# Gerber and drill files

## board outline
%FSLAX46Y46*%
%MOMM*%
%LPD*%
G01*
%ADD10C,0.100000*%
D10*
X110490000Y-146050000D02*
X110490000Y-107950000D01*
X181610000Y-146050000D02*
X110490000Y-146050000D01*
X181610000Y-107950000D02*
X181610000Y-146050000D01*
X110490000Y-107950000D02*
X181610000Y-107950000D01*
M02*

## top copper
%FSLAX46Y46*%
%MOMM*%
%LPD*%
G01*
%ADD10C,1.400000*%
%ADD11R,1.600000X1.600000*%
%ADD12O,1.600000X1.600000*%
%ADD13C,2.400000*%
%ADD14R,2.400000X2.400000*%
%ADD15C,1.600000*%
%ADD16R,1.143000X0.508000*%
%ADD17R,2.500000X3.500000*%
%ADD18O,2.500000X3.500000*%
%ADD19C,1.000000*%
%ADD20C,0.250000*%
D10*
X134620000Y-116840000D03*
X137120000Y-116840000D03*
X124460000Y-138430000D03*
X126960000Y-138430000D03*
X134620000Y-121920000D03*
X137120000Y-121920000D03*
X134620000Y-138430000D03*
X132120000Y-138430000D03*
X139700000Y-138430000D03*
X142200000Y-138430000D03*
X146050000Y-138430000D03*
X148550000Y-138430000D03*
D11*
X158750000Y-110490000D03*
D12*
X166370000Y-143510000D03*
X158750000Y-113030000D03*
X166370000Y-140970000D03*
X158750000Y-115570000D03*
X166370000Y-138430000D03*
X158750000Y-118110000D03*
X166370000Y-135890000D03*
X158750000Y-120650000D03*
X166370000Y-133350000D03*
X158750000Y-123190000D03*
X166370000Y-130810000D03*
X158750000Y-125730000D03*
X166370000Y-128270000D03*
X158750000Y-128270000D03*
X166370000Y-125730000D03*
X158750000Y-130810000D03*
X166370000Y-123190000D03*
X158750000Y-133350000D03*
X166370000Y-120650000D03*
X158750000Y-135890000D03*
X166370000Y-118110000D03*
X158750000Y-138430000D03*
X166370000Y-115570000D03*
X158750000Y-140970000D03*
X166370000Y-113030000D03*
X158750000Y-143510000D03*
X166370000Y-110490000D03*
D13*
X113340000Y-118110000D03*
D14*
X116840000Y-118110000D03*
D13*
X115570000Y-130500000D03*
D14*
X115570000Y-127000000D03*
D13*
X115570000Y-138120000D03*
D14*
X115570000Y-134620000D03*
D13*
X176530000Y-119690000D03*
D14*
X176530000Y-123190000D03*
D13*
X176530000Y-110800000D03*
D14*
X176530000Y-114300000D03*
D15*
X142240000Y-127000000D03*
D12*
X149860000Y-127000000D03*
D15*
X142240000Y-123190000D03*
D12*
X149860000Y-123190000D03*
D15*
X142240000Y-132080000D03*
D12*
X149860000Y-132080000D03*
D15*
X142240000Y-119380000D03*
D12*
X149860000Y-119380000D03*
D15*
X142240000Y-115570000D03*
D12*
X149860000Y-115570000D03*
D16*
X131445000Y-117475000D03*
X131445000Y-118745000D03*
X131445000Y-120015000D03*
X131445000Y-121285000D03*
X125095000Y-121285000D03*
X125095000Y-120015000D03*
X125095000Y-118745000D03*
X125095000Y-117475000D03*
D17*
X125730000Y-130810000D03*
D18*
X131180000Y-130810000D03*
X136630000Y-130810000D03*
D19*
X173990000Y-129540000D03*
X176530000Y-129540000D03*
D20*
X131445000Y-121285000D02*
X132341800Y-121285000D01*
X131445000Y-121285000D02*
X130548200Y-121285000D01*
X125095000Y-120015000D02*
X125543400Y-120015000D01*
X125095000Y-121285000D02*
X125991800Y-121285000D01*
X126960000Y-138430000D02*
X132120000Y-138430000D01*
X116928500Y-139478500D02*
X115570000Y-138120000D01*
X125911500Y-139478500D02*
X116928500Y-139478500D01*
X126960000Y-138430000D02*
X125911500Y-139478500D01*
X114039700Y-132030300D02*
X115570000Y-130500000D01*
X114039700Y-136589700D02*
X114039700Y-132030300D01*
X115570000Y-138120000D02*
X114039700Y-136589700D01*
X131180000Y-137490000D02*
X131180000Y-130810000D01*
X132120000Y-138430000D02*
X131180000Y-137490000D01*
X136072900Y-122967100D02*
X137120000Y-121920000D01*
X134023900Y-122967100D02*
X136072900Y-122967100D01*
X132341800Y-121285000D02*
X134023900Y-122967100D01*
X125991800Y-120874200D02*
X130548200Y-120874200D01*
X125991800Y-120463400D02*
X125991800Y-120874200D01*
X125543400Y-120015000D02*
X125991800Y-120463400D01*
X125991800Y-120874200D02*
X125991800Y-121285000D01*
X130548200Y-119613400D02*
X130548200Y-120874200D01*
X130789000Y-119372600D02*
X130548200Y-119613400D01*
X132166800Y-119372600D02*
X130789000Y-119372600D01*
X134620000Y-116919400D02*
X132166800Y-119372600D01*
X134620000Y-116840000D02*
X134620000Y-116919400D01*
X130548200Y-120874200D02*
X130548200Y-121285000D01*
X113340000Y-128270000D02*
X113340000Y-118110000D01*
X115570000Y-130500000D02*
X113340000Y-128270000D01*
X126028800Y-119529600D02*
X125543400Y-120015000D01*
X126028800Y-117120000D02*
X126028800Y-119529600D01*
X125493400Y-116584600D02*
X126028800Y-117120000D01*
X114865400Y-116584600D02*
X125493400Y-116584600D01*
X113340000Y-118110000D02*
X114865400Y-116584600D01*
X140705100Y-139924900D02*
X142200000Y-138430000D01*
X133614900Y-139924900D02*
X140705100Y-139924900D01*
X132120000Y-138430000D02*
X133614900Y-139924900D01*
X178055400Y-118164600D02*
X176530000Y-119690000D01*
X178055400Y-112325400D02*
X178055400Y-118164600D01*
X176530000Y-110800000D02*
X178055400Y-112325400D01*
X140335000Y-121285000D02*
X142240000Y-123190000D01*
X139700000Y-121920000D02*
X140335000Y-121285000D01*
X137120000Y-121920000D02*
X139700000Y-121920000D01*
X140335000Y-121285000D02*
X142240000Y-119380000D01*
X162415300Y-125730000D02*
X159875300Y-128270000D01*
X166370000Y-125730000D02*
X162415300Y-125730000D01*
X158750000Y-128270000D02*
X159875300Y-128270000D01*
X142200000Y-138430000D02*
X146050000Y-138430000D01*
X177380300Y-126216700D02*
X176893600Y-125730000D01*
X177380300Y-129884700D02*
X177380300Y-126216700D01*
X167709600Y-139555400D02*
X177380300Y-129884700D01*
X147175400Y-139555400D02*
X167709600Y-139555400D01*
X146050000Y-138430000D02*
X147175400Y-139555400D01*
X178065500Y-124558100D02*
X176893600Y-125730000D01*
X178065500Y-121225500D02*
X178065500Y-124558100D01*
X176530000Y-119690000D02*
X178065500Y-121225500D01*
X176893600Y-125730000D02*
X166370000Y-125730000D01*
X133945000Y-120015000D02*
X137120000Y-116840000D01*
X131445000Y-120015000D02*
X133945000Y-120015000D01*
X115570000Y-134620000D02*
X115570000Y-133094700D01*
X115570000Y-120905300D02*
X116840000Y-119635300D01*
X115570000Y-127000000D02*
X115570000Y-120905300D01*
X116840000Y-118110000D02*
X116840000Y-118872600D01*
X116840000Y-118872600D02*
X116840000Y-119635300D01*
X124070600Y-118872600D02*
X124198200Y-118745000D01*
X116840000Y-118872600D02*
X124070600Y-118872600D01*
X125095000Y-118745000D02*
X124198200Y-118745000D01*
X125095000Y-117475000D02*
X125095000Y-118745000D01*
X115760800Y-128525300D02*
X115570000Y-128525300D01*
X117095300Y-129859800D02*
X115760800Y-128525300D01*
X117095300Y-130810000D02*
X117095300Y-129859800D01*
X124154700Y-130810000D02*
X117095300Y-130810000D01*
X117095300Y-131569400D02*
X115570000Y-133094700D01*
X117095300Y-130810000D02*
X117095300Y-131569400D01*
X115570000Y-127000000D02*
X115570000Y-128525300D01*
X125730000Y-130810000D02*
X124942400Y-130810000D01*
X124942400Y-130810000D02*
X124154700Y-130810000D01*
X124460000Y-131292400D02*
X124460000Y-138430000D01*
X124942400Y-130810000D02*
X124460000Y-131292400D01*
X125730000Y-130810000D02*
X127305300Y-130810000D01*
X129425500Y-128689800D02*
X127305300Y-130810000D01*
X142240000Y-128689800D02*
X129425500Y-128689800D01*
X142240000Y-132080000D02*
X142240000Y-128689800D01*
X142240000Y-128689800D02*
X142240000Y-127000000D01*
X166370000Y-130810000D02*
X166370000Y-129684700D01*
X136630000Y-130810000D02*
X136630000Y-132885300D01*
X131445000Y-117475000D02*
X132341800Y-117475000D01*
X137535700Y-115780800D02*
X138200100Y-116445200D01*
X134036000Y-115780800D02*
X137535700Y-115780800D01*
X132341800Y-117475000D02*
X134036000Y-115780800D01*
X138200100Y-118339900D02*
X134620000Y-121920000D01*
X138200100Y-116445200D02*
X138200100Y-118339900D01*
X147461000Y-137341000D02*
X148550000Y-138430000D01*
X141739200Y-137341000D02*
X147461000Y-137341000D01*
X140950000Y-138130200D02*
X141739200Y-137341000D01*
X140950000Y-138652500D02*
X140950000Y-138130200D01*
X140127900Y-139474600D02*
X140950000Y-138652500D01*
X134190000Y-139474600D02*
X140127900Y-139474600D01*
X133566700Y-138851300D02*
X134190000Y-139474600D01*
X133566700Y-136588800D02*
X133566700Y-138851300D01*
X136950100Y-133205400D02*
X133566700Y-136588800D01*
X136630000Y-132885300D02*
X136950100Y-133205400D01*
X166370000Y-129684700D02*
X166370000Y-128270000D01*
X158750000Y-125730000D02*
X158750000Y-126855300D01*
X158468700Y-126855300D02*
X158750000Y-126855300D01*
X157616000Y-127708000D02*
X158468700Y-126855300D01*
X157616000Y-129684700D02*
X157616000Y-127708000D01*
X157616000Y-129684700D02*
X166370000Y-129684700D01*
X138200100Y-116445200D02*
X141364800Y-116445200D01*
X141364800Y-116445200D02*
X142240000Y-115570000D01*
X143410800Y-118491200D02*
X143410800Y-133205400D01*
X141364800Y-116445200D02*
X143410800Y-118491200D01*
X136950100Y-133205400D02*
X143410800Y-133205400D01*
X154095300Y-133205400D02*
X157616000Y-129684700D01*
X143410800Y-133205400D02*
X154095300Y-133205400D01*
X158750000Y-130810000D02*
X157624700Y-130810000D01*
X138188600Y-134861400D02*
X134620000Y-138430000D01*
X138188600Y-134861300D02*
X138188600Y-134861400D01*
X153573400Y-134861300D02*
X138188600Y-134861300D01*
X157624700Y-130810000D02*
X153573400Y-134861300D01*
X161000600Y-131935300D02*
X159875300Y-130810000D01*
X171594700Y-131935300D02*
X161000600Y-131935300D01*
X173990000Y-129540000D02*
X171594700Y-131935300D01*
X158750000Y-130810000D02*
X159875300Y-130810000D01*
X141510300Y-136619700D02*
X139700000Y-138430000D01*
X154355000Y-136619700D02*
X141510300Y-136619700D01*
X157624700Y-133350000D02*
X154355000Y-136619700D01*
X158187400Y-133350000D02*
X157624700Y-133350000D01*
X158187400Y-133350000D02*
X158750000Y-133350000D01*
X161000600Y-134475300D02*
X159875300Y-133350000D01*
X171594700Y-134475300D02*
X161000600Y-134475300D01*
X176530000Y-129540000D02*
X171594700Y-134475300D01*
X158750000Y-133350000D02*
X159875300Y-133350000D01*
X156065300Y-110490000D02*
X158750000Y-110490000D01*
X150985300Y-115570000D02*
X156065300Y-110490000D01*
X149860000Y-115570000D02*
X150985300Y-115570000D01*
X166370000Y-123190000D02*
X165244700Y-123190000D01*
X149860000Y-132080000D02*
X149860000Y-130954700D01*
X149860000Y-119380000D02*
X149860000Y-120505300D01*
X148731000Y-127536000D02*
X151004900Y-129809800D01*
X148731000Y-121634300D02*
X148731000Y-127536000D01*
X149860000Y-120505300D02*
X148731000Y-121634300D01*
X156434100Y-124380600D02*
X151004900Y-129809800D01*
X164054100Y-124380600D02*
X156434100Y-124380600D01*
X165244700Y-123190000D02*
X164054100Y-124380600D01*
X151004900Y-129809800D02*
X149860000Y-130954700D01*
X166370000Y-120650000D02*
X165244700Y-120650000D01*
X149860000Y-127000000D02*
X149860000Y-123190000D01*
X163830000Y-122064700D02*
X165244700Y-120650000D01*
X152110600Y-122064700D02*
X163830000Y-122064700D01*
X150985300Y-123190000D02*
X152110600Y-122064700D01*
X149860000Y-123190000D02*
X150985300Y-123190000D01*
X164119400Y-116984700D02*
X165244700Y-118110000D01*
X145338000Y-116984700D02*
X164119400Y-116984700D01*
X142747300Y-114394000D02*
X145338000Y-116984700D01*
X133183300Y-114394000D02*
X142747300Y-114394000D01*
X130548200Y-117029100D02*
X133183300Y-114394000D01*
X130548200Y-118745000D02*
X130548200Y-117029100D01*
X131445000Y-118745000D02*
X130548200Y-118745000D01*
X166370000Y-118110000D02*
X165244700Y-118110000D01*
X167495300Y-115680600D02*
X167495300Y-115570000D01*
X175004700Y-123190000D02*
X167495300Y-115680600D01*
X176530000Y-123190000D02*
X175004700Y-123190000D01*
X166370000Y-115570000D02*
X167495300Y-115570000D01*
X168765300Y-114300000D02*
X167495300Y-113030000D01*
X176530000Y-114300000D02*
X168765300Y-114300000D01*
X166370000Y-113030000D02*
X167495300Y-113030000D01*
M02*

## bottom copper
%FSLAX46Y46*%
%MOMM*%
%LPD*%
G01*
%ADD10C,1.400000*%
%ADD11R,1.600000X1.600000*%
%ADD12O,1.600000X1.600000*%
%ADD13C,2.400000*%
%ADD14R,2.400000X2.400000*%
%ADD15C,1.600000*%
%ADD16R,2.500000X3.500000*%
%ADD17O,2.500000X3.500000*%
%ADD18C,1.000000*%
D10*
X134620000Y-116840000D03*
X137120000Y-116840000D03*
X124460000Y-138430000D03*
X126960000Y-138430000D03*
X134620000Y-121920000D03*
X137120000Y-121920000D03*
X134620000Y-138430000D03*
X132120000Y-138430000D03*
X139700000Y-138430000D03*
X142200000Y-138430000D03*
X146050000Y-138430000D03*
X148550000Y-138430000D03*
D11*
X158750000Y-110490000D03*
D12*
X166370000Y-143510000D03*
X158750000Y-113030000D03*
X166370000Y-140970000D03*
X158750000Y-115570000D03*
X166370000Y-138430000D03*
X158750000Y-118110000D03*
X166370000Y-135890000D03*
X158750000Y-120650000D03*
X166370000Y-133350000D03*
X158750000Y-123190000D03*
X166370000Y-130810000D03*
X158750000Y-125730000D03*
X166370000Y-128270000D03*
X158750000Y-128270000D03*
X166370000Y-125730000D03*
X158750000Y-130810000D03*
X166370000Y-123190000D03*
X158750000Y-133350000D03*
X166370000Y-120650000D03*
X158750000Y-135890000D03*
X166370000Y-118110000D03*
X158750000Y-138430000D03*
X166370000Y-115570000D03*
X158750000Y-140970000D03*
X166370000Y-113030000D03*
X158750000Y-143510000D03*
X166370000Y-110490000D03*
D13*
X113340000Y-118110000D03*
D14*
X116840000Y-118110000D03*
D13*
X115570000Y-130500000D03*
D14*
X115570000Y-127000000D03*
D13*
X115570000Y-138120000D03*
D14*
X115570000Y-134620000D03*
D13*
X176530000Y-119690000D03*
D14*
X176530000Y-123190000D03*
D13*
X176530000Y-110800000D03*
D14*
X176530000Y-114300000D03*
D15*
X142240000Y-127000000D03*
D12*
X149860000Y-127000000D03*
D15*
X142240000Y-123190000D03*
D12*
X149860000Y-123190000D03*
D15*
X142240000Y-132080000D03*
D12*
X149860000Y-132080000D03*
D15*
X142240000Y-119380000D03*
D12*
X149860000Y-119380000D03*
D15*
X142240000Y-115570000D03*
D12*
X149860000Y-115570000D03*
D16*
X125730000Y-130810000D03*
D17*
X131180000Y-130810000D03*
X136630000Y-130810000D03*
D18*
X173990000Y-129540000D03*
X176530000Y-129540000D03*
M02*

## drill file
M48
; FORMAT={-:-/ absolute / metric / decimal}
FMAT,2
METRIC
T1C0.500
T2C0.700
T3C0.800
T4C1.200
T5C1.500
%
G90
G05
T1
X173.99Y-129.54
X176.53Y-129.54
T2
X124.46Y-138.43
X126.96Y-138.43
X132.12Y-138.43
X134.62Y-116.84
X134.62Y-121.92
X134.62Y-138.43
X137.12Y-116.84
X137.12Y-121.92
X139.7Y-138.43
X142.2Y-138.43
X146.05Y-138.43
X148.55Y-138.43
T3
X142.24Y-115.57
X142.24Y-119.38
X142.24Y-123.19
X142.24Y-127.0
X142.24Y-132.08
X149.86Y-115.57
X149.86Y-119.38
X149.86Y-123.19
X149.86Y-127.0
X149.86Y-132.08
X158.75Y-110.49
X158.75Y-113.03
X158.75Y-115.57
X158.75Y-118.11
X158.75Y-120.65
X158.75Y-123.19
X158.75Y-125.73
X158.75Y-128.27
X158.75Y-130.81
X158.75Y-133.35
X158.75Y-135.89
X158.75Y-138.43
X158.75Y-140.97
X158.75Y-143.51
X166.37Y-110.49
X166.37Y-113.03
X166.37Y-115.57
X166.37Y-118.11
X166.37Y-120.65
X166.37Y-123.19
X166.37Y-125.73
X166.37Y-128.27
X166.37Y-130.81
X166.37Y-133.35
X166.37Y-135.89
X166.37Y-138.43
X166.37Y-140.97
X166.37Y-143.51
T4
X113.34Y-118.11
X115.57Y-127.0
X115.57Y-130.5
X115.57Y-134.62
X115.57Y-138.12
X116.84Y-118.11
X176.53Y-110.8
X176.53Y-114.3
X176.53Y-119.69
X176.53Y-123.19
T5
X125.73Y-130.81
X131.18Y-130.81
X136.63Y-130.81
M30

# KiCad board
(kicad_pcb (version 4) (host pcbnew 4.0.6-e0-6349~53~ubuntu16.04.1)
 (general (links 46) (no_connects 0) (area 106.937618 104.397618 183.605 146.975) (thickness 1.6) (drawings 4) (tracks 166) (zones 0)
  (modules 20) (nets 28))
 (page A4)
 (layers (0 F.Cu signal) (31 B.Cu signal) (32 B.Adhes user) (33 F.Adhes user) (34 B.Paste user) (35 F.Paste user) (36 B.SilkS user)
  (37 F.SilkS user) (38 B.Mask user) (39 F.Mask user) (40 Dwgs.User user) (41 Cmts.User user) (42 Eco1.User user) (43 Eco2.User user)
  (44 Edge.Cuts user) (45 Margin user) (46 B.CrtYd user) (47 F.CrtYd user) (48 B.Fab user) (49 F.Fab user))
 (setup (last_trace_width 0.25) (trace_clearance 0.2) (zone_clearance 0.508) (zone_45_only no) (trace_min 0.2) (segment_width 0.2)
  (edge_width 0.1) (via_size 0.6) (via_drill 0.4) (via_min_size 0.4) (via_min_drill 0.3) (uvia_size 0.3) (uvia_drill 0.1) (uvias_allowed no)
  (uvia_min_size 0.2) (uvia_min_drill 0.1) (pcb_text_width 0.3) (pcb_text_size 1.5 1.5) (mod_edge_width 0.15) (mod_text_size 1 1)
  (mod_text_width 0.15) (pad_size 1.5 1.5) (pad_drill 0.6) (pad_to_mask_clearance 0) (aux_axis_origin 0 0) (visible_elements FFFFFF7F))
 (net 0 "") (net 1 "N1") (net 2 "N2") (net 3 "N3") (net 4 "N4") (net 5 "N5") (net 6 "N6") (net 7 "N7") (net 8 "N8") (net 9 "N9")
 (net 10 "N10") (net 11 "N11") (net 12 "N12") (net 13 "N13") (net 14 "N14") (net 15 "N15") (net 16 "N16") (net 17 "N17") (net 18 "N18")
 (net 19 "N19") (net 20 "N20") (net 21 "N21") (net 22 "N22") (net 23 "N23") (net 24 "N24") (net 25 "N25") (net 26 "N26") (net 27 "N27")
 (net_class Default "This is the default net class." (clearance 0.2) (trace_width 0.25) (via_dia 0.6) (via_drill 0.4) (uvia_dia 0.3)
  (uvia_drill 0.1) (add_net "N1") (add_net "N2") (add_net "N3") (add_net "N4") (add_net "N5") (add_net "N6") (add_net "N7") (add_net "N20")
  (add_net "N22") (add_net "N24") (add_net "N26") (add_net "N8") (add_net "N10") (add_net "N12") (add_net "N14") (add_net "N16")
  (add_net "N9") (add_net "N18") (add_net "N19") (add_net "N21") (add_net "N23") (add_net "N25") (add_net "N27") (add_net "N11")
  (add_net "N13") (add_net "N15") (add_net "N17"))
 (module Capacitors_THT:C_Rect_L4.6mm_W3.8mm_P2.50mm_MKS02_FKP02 (layer F.Cu) (at 134.62 116.84)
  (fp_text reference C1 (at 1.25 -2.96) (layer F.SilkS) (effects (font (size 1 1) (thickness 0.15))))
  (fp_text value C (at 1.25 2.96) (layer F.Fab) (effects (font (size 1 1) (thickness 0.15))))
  (pad 1 thru_hole circle (at 0 0) (size 1.4 1.4) (drill 0.7) (layers *.Cu *.Mask) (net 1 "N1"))
  (pad 2 thru_hole circle (at 2.5 0) (size 1.4 1.4) (drill 0.7) (layers *.Cu *.Mask) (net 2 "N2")))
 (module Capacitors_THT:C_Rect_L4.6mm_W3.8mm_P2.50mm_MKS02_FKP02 (layer F.Cu) (at 124.46 138.43)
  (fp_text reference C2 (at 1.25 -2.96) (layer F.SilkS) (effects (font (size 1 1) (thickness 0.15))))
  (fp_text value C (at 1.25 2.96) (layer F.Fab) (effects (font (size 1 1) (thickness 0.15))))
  (pad 1 thru_hole circle (at 0 0) (size 1.4 1.4) (drill 0.7) (layers *.Cu *.Mask) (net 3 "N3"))
  (pad 2 thru_hole circle (at 2.5 0) (size 1.4 1.4) (drill 0.7) (layers *.Cu *.Mask) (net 1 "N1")))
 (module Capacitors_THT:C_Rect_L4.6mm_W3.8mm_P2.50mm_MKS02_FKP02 (layer F.Cu) (at 134.62 121.92)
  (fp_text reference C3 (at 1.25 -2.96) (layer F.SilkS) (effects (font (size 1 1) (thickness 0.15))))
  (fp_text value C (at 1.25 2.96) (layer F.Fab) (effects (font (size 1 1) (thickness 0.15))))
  (pad 1 thru_hole circle (at 0 0) (size 1.4 1.4) (drill 0.7) (layers *.Cu *.Mask) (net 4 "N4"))
  (pad 2 thru_hole circle (at 2.5 0) (size 1.4 1.4) (drill 0.7) (layers *.Cu *.Mask) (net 1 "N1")))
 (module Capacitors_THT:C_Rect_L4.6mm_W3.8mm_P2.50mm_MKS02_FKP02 (layer F.Cu) (at 134.62 138.43 180)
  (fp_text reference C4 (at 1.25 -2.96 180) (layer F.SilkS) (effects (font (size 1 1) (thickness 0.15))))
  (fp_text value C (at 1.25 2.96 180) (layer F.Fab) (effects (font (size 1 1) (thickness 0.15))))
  (pad 1 thru_hole circle (at 0 0 180) (size 1.4 1.4) (drill 0.7) (layers *.Cu *.Mask) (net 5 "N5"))
  (pad 2 thru_hole circle (at 2.5 0 180) (size 1.4 1.4) (drill 0.7) (layers *.Cu *.Mask) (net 1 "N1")))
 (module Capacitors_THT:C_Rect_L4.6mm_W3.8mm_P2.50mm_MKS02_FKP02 (layer F.Cu) (at 139.7 138.43)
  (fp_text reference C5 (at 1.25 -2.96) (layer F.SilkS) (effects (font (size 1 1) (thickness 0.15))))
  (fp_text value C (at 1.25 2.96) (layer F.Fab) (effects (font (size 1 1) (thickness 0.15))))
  (pad 1 thru_hole circle (at 0 0) (size 1.4 1.4) (drill 0.7) (layers *.Cu *.Mask) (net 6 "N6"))
  (pad 2 thru_hole circle (at 2.5 0) (size 1.4 1.4) (drill 0.7) (layers *.Cu *.Mask) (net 1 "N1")))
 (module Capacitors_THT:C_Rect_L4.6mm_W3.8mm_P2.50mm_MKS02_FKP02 (layer F.Cu) (at 146.05 138.43)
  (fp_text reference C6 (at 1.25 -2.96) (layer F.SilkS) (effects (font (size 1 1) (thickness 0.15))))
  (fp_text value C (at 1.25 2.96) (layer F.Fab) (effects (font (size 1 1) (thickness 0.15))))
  (pad 1 thru_hole circle (at 0 0) (size 1.4 1.4) (drill 0.7) (layers *.Cu *.Mask) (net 1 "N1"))
  (pad 2 thru_hole circle (at 2.5 0) (size 1.4 1.4) (drill 0.7) (layers *.Cu *.Mask) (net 4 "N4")))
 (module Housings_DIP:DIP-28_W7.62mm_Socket (layer F.Cu) (at 158.75 110.49)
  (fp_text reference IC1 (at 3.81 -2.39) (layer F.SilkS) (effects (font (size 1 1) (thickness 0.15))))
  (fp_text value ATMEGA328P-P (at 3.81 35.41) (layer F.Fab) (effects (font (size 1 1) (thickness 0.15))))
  (pad 1 thru_hole rect (at 0 0) (size 1.6 1.6) (drill 0.8) (layers *.Cu *.Mask) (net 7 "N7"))
  (pad 15 thru_hole oval (at 7.62 33.02) (size 1.6 1.6) (drill 0.8) (layers *.Cu *.Mask) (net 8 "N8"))
  (pad 2 thru_hole oval (at 0 2.54) (size 1.6 1.6) (drill 0.8) (layers *.Cu *.Mask) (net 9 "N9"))
  (pad 16 thru_hole oval (at 7.62 30.48) (size 1.6 1.6) (drill 0.8) (layers *.Cu *.Mask) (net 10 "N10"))
  (pad 3 thru_hole oval (at 0 5.08) (size 1.6 1.6) (drill 0.8) (layers *.Cu *.Mask) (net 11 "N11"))
  (pad 17 thru_hole oval (at 7.62 27.94) (size 1.6 1.6) (drill 0.8) (layers *.Cu *.Mask) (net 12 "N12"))
  (pad 4 thru_hole oval (at 0 7.62) (size 1.6 1.6) (drill 0.8) (layers *.Cu *.Mask) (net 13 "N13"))
  (pad 18 thru_hole oval (at 7.62 25.4) (size 1.6 1.6) (drill 0.8) (layers *.Cu *.Mask) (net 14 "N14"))
  (pad 5 thru_hole oval (at 0 10.16) (size 1.6 1.6) (drill 0.8) (layers *.Cu *.Mask) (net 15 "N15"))
  (pad 19 thru_hole oval (at 7.62 22.86) (size 1.6 1.6) (drill 0.8) (layers *.Cu *.Mask) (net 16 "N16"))
  (pad 6 thru_hole oval (at 0 12.7) (size 1.6 1.6) (drill 0.8) (layers *.Cu *.Mask) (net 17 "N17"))
  (pad 20 thru_hole oval (at 7.62 20.32) (size 1.6 1.6) (drill 0.8) (layers *.Cu *.Mask) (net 4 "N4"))
  (pad 7 thru_hole oval (at 0 15.24) (size 1.6 1.6) (drill 0.8) (layers *.Cu *.Mask) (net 4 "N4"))
  (pad 21 thru_hole oval (at 7.62 17.78) (size 1.6 1.6) (drill 0.8) (layers *.Cu *.Mask) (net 4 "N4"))
  (pad 8 thru_hole oval (at 0 17.78) (size 1.6 1.6) (drill 0.8) (layers *.Cu *.Mask) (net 1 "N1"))
  (pad 22 thru_hole oval (at 7.62 15.24) (size 1.6 1.6) (drill 0.8) (layers *.Cu *.Mask) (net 1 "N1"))
  (pad 9 thru_hole oval (at 0 20.32) (size 1.6 1.6) (drill 0.8) (layers *.Cu *.Mask) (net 5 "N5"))
  (pad 23 thru_hole oval (at 7.62 12.7) (size 1.6 1.6) (drill 0.8) (layers *.Cu *.Mask) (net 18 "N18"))
  (pad 10 thru_hole oval (at 0 22.86) (size 1.6 1.6) (drill 0.8) (layers *.Cu *.Mask) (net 6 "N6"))
  (pad 24 thru_hole oval (at 7.62 10.16) (size 1.6 1.6) (drill 0.8) (layers *.Cu *.Mask) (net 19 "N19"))
  (pad 11 thru_hole oval (at 0 25.4) (size 1.6 1.6) (drill 0.8) (layers *.Cu *.Mask) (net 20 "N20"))
  (pad 25 thru_hole oval (at 7.62 7.62) (size 1.6 1.6) (drill 0.8) (layers *.Cu *.Mask) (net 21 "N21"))
  (pad 12 thru_hole oval (at 0 27.94) (size 1.6 1.6) (drill 0.8) (layers *.Cu *.Mask) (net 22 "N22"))
  (pad 26 thru_hole oval (at 7.62 5.08) (size 1.6 1.6) (drill 0.8) (layers *.Cu *.Mask) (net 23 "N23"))
  (pad 13 thru_hole oval (at 0 30.48) (size 1.6 1.6) (drill 0.8) (layers *.Cu *.Mask) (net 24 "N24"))
  (pad 27 thru_hole oval (at 7.62 2.54) (size 1.6 1.6) (drill 0.8) (layers *.Cu *.Mask) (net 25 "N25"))
  (pad 14 thru_hole oval (at 0 33.02) (size 1.6 1.6) (drill 0.8) (layers *.Cu *.Mask) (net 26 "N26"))
  (pad 28 thru_hole oval (at 7.62 0) (size 1.6 1.6) (drill 0.8) (layers *.Cu *.Mask) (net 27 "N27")))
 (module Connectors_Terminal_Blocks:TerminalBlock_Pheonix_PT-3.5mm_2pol (layer F.Cu) (at 116.84 118.11 180)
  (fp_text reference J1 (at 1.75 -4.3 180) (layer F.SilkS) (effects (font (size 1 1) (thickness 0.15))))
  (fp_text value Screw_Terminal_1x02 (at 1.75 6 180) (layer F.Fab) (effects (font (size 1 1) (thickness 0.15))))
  (pad 2 thru_hole circle (at 3.5 0 180) (size 2.4 2.4) (drill 1.2) (layers *.Cu *.Mask) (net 1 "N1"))
  (pad 1 thru_hole rect (at 0 0 180) (size 2.4 2.4) (drill 1.2) (layers *.Cu *.Mask) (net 3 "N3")))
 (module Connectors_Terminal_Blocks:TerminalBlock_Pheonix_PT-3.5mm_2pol (layer F.Cu) (at 115.57 127 270)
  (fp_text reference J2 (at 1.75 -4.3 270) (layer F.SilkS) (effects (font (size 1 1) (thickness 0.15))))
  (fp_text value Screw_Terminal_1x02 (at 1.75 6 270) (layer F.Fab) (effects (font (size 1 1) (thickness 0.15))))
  (pad 2 thru_hole circle (at 3.5 0 270) (size 2.4 2.4) (drill 1.2) (layers *.Cu *.Mask) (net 1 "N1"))
  (pad 1 thru_hole rect (at 0 0 270) (size 2.4 2.4) (drill 1.2) (layers *.Cu *.Mask) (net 3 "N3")))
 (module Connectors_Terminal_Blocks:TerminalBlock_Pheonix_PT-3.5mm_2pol (layer F.Cu) (at 115.57 134.62 270)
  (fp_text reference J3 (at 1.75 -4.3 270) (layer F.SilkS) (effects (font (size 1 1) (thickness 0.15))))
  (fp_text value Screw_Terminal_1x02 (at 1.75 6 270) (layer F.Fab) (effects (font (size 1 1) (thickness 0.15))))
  (pad 2 thru_hole circle (at 3.5 0 270) (size 2.4 2.4) (drill 1.2) (layers *.Cu *.Mask) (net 1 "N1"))
  (pad 1 thru_hole rect (at 0 0 270) (size 2.4 2.4) (drill 1.2) (layers *.Cu *.Mask) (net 3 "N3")))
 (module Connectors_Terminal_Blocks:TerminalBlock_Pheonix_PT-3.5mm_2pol (layer F.Cu) (at 176.53 123.19 90)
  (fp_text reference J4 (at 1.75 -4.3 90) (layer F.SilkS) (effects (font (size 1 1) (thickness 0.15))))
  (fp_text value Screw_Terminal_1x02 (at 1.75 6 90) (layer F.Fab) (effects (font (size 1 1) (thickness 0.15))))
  (pad 2 thru_hole circle (at 3.5 0 90) (size 2.4 2.4) (drill 1.2) (layers *.Cu *.Mask) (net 1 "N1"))
  (pad 1 thru_hole rect (at 0 0 90) (size 2.4 2.4) (drill 1.2) (layers *.Cu *.Mask) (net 23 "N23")))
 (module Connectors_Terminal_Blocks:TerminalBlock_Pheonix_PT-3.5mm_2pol (layer F.Cu) (at 176.53 114.3 90)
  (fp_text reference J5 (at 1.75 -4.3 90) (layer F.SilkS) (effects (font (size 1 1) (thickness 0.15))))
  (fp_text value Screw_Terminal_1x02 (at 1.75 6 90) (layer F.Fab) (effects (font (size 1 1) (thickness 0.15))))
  (pad 2 thru_hole circle (at 3.5 0 90) (size 2.4 2.4) (drill 1.2) (layers *.Cu *.Mask) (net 1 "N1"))
  (pad 1 thru_hole rect (at 0 0 90) (size 2.4 2.4) (drill 1.2) (layers *.Cu *.Mask) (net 25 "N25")))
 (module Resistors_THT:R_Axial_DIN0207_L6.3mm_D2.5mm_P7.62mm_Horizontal (layer F.Cu) (at 142.24 127)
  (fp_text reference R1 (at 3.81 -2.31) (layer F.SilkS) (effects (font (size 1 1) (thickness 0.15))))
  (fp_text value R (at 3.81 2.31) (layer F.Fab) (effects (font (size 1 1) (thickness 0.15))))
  (pad 1 thru_hole circle (at 0 0) (size 1.6 1.6) (drill 0.8) (layers *.Cu *.Mask) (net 3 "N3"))
  (pad 2 thru_hole oval (at 7.62 0) (size 1.6 1.6) (drill 0.8) (layers *.Cu *.Mask) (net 19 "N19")))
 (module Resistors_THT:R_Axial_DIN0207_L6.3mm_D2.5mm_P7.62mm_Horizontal (layer F.Cu) (at 142.24 123.19)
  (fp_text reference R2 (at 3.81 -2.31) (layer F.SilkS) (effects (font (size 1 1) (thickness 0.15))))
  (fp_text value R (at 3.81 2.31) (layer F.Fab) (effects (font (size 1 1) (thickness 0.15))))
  (pad 1 thru_hole circle (at 0 0) (size 1.6 1.6) (drill 0.8) (layers *.Cu *.Mask) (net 1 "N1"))
  (pad 2 thru_hole oval (at 7.62 0) (size 1.6 1.6) (drill 0.8) (layers *.Cu *.Mask) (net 19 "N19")))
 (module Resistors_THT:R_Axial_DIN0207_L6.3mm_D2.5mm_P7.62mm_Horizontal (layer F.Cu) (at 142.24 132.08)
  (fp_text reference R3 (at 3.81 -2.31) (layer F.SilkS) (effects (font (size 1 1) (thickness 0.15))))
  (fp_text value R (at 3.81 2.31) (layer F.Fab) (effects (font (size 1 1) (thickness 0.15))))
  (pad 1 thru_hole circle (at 0 0) (size 1.6 1.6) (drill 0.8) (layers *.Cu *.Mask) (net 3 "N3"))
  (pad 2 thru_hole oval (at 7.62 0) (size 1.6 1.6) (drill 0.8) (layers *.Cu *.Mask) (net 18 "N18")))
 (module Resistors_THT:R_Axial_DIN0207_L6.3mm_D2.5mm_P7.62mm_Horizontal (layer F.Cu) (at 142.24 119.38)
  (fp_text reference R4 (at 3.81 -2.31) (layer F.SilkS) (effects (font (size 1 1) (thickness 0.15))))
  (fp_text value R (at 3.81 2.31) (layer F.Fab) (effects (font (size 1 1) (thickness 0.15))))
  (pad 1 thru_hole circle (at 0 0) (size 1.6 1.6) (drill 0.8) (layers *.Cu *.Mask) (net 1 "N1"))
  (pad 2 thru_hole oval (at 7.62 0) (size 1.6 1.6) (drill 0.8) (layers *.Cu *.Mask) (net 18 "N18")))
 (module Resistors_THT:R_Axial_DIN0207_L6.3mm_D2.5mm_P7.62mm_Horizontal (layer F.Cu) (at 142.24 115.57)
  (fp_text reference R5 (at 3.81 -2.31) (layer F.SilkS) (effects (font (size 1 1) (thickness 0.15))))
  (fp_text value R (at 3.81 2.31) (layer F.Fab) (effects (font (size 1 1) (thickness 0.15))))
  (pad 1 thru_hole circle (at 0 0) (size 1.6 1.6) (drill 0.8) (layers *.Cu *.Mask) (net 4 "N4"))
  (pad 2 thru_hole oval (at 7.62 0) (size 1.6 1.6) (drill 0.8) (layers *.Cu *.Mask) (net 7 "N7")))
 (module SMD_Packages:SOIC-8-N (layer F.Cu) (at 128.27 119.38 270)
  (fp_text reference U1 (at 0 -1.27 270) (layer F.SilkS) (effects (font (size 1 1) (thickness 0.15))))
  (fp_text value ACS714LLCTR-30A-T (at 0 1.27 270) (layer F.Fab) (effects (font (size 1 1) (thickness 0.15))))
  (pad 8 smd rect (at -1.905 -3.175 270) (size 0.508 1.143) (layers F.Cu F.Paste F.Mask) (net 4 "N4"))
  (pad 7 smd rect (at -0.635 -3.175 270) (size 0.508 1.143) (layers F.Cu F.Paste F.Mask) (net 21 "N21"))
  (pad 6 smd rect (at 0.635 -3.175 270) (size 0.508 1.143) (layers F.Cu F.Paste F.Mask) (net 2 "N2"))
  (pad 5 smd rect (at 1.905 -3.175 270) (size 0.508 1.143) (layers F.Cu F.Paste F.Mask) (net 1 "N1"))
  (pad 4 smd rect (at 1.905 3.175 270) (size 0.508 1.143) (layers F.Cu F.Paste F.Mask) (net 1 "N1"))
  (pad 3 smd rect (at 0.635 3.175 270) (size 0.508 1.143) (layers F.Cu F.Paste F.Mask) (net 1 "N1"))
  (pad 2 smd rect (at -0.635 3.175 270) (size 0.508 1.143) (layers F.Cu F.Paste F.Mask) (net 3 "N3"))
  (pad 1 smd rect (at -1.905 3.175 270) (size 0.508 1.143) (layers F.Cu F.Paste F.Mask) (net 3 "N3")))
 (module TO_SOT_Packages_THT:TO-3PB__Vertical (layer F.Cu) (at 125.73 130.81)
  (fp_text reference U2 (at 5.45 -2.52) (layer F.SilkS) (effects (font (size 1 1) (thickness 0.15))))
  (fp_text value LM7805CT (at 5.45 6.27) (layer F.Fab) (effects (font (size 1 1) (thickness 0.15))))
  (pad 1 thru_hole rect (at 0 0) (size 2.5 3.5) (drill 1.5) (layers *.Cu *.Mask) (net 3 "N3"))
  (pad 2 thru_hole oval (at 5.45 0) (size 2.5 3.5) (drill 1.5) (layers *.Cu *.Mask) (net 1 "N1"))
  (pad 3 thru_hole oval (at 10.9 0) (size 2.5 3.5) (drill 1.5) (layers *.Cu *.Mask) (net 4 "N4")))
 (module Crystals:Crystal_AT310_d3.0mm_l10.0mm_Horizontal (layer F.Cu) (at 173.99 129.54)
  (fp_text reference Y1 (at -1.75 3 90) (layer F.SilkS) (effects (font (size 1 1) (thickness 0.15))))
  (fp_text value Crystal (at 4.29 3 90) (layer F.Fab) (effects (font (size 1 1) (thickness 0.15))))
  (pad 1 thru_hole circle (at 0 0) (size 1 1) (drill 0.5) (layers *.Cu *.Mask) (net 5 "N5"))
  (pad 2 thru_hole circle (at 2.54 0) (size 1 1) (drill 0.5) (layers *.Cu *.Mask) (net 6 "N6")))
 (gr_line (start 110.49 146.05) (end 110.49 107.95) (angle 90) (layer Edge.Cuts) (width 0.1))
 (gr_line (start 181.61 146.05) (end 110.49 146.05) (angle 90) (layer Edge.Cuts) (width 0.1))
 (gr_line (start 181.61 107.95) (end 181.61 146.05) (angle 90) (layer Edge.Cuts) (width 0.1))
 (gr_line (start 110.49 107.95) (end 181.61 107.95) (angle 90) (layer Edge.Cuts) (width 0.1))
 (segment (start 131.445 121.285) (end 132.3418 121.285) (width 0.25) (layer F.Cu) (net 1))
 (segment (start 131.445 121.285) (end 130.5482 121.285) (width 0.25) (layer F.Cu) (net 1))
 (segment (start 125.095 120.015) (end 125.5434 120.015) (width 0.25) (layer F.Cu) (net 1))
 (segment (start 125.095 121.285) (end 125.9918 121.285) (width 0.25) (layer F.Cu) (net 1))
 (segment (start 126.96 138.43) (end 132.12 138.43) (width 0.25) (layer F.Cu) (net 1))
 (segment (start 116.9285 139.4785) (end 115.57 138.12) (width 0.25) (layer F.Cu) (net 1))
 (segment (start 125.9115 139.4785) (end 116.9285 139.4785) (width 0.25) (layer F.Cu) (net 1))
 (segment (start 126.96 138.43) (end 125.9115 139.4785) (width 0.25) (layer F.Cu) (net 1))
 (segment (start 114.0397 132.0303) (end 115.57 130.5) (width 0.25) (layer F.Cu) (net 1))
 (segment (start 114.0397 136.5897) (end 114.0397 132.0303) (width 0.25) (layer F.Cu) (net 1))
 (segment (start 115.57 138.12) (end 114.0397 136.5897) (width 0.25) (layer F.Cu) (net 1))
 (segment (start 131.18 137.49) (end 131.18 130.81) (width 0.25) (layer F.Cu) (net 1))
 (segment (start 132.12 138.43) (end 131.18 137.49) (width 0.25) (layer F.Cu) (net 1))
 (segment (start 136.0729 122.9671) (end 137.12 121.92) (width 0.25) (layer F.Cu) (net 1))
 (segment (start 134.0239 122.9671) (end 136.0729 122.9671) (width 0.25) (layer F.Cu) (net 1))
 (segment (start 132.3418 121.285) (end 134.0239 122.9671) (width 0.25) (layer F.Cu) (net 1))
 (segment (start 125.9918 120.8742) (end 130.5482 120.8742) (width 0.25) (layer F.Cu) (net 1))
 (segment (start 125.9918 120.4634) (end 125.9918 120.8742) (width 0.25) (layer F.Cu) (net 1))
 (segment (start 125.5434 120.015) (end 125.9918 120.4634) (width 0.25) (layer F.Cu) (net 1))
 (segment (start 125.9918 120.8742) (end 125.9918 121.285) (width 0.25) (layer F.Cu) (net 1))
 (segment (start 130.5482 119.6134) (end 130.5482 120.8742) (width 0.25) (layer F.Cu) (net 1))
 (segment (start 130.789 119.3726) (end 130.5482 119.6134) (width 0.25) (layer F.Cu) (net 1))
 (segment (start 132.1668 119.3726) (end 130.789 119.3726) (width 0.25) (layer F.Cu) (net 1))
 (segment (start 134.62 116.9194) (end 132.1668 119.3726) (width 0.25) (layer F.Cu) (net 1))
 (segment (start 134.62 116.84) (end 134.62 116.9194) (width 0.25) (layer F.Cu) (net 1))
 (segment (start 130.5482 120.8742) (end 130.5482 121.285) (width 0.25) (layer F.Cu) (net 1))
 (segment (start 113.34 128.27) (end 113.34 118.11) (width 0.25) (layer F.Cu) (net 1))
 (segment (start 115.57 130.5) (end 113.34 128.27) (width 0.25) (layer F.Cu) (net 1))
 (segment (start 126.0288 119.5296) (end 125.5434 120.015) (width 0.25) (layer F.Cu) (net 1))
 (segment (start 126.0288 117.12) (end 126.0288 119.5296) (width 0.25) (layer F.Cu) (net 1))
 (segment (start 125.4934 116.5846) (end 126.0288 117.12) (width 0.25) (layer F.Cu) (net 1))
 (segment (start 114.8654 116.5846) (end 125.4934 116.5846) (width 0.25) (layer F.Cu) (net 1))
 (segment (start 113.34 118.11) (end 114.8654 116.5846) (width 0.25) (layer F.Cu) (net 1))
 (segment (start 140.7051 139.9249) (end 142.2 138.43) (width 0.25) (layer F.Cu) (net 1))
 (segment (start 133.6149 139.9249) (end 140.7051 139.9249) (width 0.25) (layer F.Cu) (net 1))
 (segment (start 132.12 138.43) (end 133.6149 139.9249) (width 0.25) (layer F.Cu) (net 1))
 (segment (start 178.0554 118.1646) (end 176.53 119.69) (width 0.25) (layer F.Cu) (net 1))
 (segment (start 178.0554 112.3254) (end 178.0554 118.1646) (width 0.25) (layer F.Cu) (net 1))
 (segment (start 176.53 110.8) (end 178.0554 112.3254) (width 0.25) (layer F.Cu) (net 1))
 (segment (start 140.335 121.285) (end 142.24 123.19) (width 0.25) (layer F.Cu) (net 1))
 (segment (start 139.7 121.92) (end 140.335 121.285) (width 0.25) (layer F.Cu) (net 1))
 (segment (start 137.12 121.92) (end 139.7 121.92) (width 0.25) (layer F.Cu) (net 1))
 (segment (start 140.335 121.285) (end 142.24 119.38) (width 0.25) (layer F.Cu) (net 1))
 (segment (start 162.4153 125.73) (end 159.8753 128.27) (width 0.25) (layer F.Cu) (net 1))
 (segment (start 166.37 125.73) (end 162.4153 125.73) (width 0.25) (layer F.Cu) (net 1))
 (segment (start 158.75 128.27) (end 159.8753 128.27) (width 0.25) (layer F.Cu) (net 1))
 (segment (start 142.2 138.43) (end 146.05 138.43) (width 0.25) (layer F.Cu) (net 1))
 (segment (start 177.3803 126.2167) (end 176.8936 125.73) (width 0.25) (layer F.Cu) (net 1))
 (segment (start 177.3803 129.8847) (end 177.3803 126.2167) (width 0.25) (layer F.Cu) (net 1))
 (segment (start 167.7096 139.5554) (end 177.3803 129.8847) (width 0.25) (layer F.Cu) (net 1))
 (segment (start 147.1754 139.5554) (end 167.7096 139.5554) (width 0.25) (layer F.Cu) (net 1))
 (segment (start 146.05 138.43) (end 147.1754 139.5554) (width 0.25) (layer F.Cu) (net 1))
 (segment (start 178.0655 124.5581) (end 176.8936 125.73) (width 0.25) (layer F.Cu) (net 1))
 (segment (start 178.0655 121.2255) (end 178.0655 124.5581) (width 0.25) (layer F.Cu) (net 1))
 (segment (start 176.53 119.69) (end 178.0655 121.2255) (width 0.25) (layer F.Cu) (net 1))
 (segment (start 176.8936 125.73) (end 166.37 125.73) (width 0.25) (layer F.Cu) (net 1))
 (segment (start 133.945 120.015) (end 137.12 116.84) (width 0.25) (layer F.Cu) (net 2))
 (segment (start 131.445 120.015) (end 133.945 120.015) (width 0.25) (layer F.Cu) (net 2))
 (segment (start 115.57 134.62) (end 115.57 133.0947) (width 0.25) (layer F.Cu) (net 3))
 (segment (start 115.57 120.9053) (end 116.84 119.6353) (width 0.25) (layer F.Cu) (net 3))
 (segment (start 115.57 127) (end 115.57 120.9053) (width 0.25) (layer F.Cu) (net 3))
 (segment (start 116.84 118.11) (end 116.84 118.8726) (width 0.25) (layer F.Cu) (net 3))
 (segment (start 116.84 118.8726) (end 116.84 119.6353) (width 0.25) (layer F.Cu) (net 3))
 (segment (start 124.0706 118.8726) (end 124.1982 118.745) (width 0.25) (layer F.Cu) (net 3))
 (segment (start 116.84 118.8726) (end 124.0706 118.8726) (width 0.25) (layer F.Cu) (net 3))
 (segment (start 125.095 118.745) (end 124.1982 118.745) (width 0.25) (layer F.Cu) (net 3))
 (segment (start 125.095 117.475) (end 125.095 118.745) (width 0.25) (layer F.Cu) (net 3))
 (segment (start 115.7608 128.5253) (end 115.57 128.5253) (width 0.25) (layer F.Cu) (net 3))
 (segment (start 117.0953 129.8598) (end 115.7608 128.5253) (width 0.25) (layer F.Cu) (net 3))
 (segment (start 117.0953 130.81) (end 117.0953 129.8598) (width 0.25) (layer F.Cu) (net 3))
 (segment (start 124.1547 130.81) (end 117.0953 130.81) (width 0.25) (layer F.Cu) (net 3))
 (segment (start 117.0953 131.5694) (end 115.57 133.0947) (width 0.25) (layer F.Cu) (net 3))
 (segment (start 117.0953 130.81) (end 117.0953 131.5694) (width 0.25) (layer F.Cu) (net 3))
 (segment (start 115.57 127) (end 115.57 128.5253) (width 0.25) (layer F.Cu) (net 3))
 (segment (start 125.73 130.81) (end 124.9424 130.81) (width 0.25) (layer F.Cu) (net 3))
 (segment (start 124.9424 130.81) (end 124.1547 130.81) (width 0.25) (layer F.Cu) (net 3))
 (segment (start 124.46 131.2924) (end 124.46 138.43) (width 0.25) (layer F.Cu) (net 3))
 (segment (start 124.9424 130.81) (end 124.46 131.2924) (width 0.25) (layer F.Cu) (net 3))
 (segment (start 125.73 130.81) (end 127.3053 130.81) (width 0.25) (layer F.Cu) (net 3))
 (segment (start 129.4255 128.6898) (end 127.3053 130.81) (width 0.25) (layer F.Cu) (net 3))
 (segment (start 142.24 128.6898) (end 129.4255 128.6898) (width 0.25) (layer F.Cu) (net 3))
 (segment (start 142.24 132.08) (end 142.24 128.6898) (width 0.25) (layer F.Cu) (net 3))
 (segment (start 142.24 128.6898) (end 142.24 127) (width 0.25) (layer F.Cu) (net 3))
 (segment (start 166.37 130.81) (end 166.37 129.6847) (width 0.25) (layer F.Cu) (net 4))
 (segment (start 136.63 130.81) (end 136.63 132.8853) (width 0.25) (layer F.Cu) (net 4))
 (segment (start 131.445 117.475) (end 132.3418 117.475) (width 0.25) (layer F.Cu) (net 4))
 (segment (start 137.5357 115.7808) (end 138.2001 116.4452) (width 0.25) (layer F.Cu) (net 4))
 (segment (start 134.036 115.7808) (end 137.5357 115.7808) (width 0.25) (layer F.Cu) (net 4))
 (segment (start 132.3418 117.475) (end 134.036 115.7808) (width 0.25) (layer F.Cu) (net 4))
 (segment (start 138.2001 118.3399) (end 134.62 121.92) (width 0.25) (layer F.Cu) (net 4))
 (segment (start 138.2001 116.4452) (end 138.2001 118.3399) (width 0.25) (layer F.Cu) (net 4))
 (segment (start 147.461 137.341) (end 148.55 138.43) (width 0.25) (layer F.Cu) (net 4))
 (segment (start 141.7392 137.341) (end 147.461 137.341) (width 0.25) (layer F.Cu) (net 4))
 (segment (start 140.95 138.1302) (end 141.7392 137.341) (width 0.25) (layer F.Cu) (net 4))
 (segment (start 140.95 138.6525) (end 140.95 138.1302) (width 0.25) (layer F.Cu) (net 4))
 (segment (start 140.1279 139.4746) (end 140.95 138.6525) (width 0.25) (layer F.Cu) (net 4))
 (segment (start 134.19 139.4746) (end 140.1279 139.4746) (width 0.25) (layer F.Cu) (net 4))
 (segment (start 133.5667 138.8513) (end 134.19 139.4746) (width 0.25) (layer F.Cu) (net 4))
 (segment (start 133.5667 136.5888) (end 133.5667 138.8513) (width 0.25) (layer F.Cu) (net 4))
 (segment (start 136.9501 133.2054) (end 133.5667 136.5888) (width 0.25) (layer F.Cu) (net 4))
 (segment (start 136.63 132.8853) (end 136.9501 133.2054) (width 0.25) (layer F.Cu) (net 4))
 (segment (start 166.37 129.6847) (end 166.37 128.27) (width 0.25) (layer F.Cu) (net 4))
 (segment (start 158.75 125.73) (end 158.75 126.8553) (width 0.25) (layer F.Cu) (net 4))
 (segment (start 158.4687 126.8553) (end 158.75 126.8553) (width 0.25) (layer F.Cu) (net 4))
 (segment (start 157.616 127.708) (end 158.4687 126.8553) (width 0.25) (layer F.Cu) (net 4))
 (segment (start 157.616 129.6847) (end 157.616 127.708) (width 0.25) (layer F.Cu) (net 4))
 (segment (start 157.616 129.6847) (end 166.37 129.6847) (width 0.25) (layer F.Cu) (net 4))
 (segment (start 138.2001 116.4452) (end 141.3648 116.4452) (width 0.25) (layer F.Cu) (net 4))
 (segment (start 141.3648 116.4452) (end 142.24 115.57) (width 0.25) (layer F.Cu) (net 4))
 (segment (start 143.4108 118.4912) (end 143.4108 133.2054) (width 0.25) (layer F.Cu) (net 4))
 (segment (start 141.3648 116.4452) (end 143.4108 118.4912) (width 0.25) (layer F.Cu) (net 4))
 (segment (start 136.9501 133.2054) (end 143.4108 133.2054) (width 0.25) (layer F.Cu) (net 4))
 (segment (start 154.0953 133.2054) (end 157.616 129.6847) (width 0.25) (layer F.Cu) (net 4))
 (segment (start 143.4108 133.2054) (end 154.0953 133.2054) (width 0.25) (layer F.Cu) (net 4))
 (segment (start 158.75 130.81) (end 157.6247 130.81) (width 0.25) (layer F.Cu) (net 5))
 (segment (start 138.1886 134.8614) (end 134.62 138.43) (width 0.25) (layer F.Cu) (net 5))
 (segment (start 138.1886 134.8613) (end 138.1886 134.8614) (width 0.25) (layer F.Cu) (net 5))
 (segment (start 153.5734 134.8613) (end 138.1886 134.8613) (width 0.25) (layer F.Cu) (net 5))
 (segment (start 157.6247 130.81) (end 153.5734 134.8613) (width 0.25) (layer F.Cu) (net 5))
 (segment (start 161.0006 131.9353) (end 159.8753 130.81) (width 0.25) (layer F.Cu) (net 5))
 (segment (start 171.5947 131.9353) (end 161.0006 131.9353) (width 0.25) (layer F.Cu) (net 5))
 (segment (start 173.99 129.54) (end 171.5947 131.9353) (width 0.25) (layer F.Cu) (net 5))
 (segment (start 158.75 130.81) (end 159.8753 130.81) (width 0.25) (layer F.Cu) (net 5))
 (segment (start 141.5103 136.6197) (end 139.7 138.43) (width 0.25) (layer F.Cu) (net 6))
 (segment (start 154.355 136.6197) (end 141.5103 136.6197) (width 0.25) (layer F.Cu) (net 6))
 (segment (start 157.6247 133.35) (end 154.355 136.6197) (width 0.25) (layer F.Cu) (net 6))
 (segment (start 158.1874 133.35) (end 157.6247 133.35) (width 0.25) (layer F.Cu) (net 6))
 (segment (start 158.1874 133.35) (end 158.75 133.35) (width 0.25) (layer F.Cu) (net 6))
 (segment (start 161.0006 134.4753) (end 159.8753 133.35) (width 0.25) (layer F.Cu) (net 6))
 (segment (start 171.5947 134.4753) (end 161.0006 134.4753) (width 0.25) (layer F.Cu) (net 6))
 (segment (start 176.53 129.54) (end 171.5947 134.4753) (width 0.25) (layer F.Cu) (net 6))
 (segment (start 158.75 133.35) (end 159.8753 133.35) (width 0.25) (layer F.Cu) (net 6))
 (segment (start 156.0653 110.49) (end 158.75 110.49) (width 0.25) (layer F.Cu) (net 7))
 (segment (start 150.9853 115.57) (end 156.0653 110.49) (width 0.25) (layer F.Cu) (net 7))
 (segment (start 149.86 115.57) (end 150.9853 115.57) (width 0.25) (layer F.Cu) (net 7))
 (segment (start 166.37 123.19) (end 165.2447 123.19) (width 0.25) (layer F.Cu) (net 18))
 (segment (start 149.86 132.08) (end 149.86 130.9547) (width 0.25) (layer F.Cu) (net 18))
 (segment (start 149.86 119.38) (end 149.86 120.5053) (width 0.25) (layer F.Cu) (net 18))
 (segment (start 148.731 127.536) (end 151.0049 129.8098) (width 0.25) (layer F.Cu) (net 18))
 (segment (start 148.731 121.6343) (end 148.731 127.536) (width 0.25) (layer F.Cu) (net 18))
 (segment (start 149.86 120.5053) (end 148.731 121.6343) (width 0.25) (layer F.Cu) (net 18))
 (segment (start 156.4341 124.3806) (end 151.0049 129.8098) (width 0.25) (layer F.Cu) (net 18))
 (segment (start 164.0541 124.3806) (end 156.4341 124.3806) (width 0.25) (layer F.Cu) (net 18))
 (segment (start 165.2447 123.19) (end 164.0541 124.3806) (width 0.25) (layer F.Cu) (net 18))
 (segment (start 151.0049 129.8098) (end 149.86 130.9547) (width 0.25) (layer F.Cu) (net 18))
 (segment (start 166.37 120.65) (end 165.2447 120.65) (width 0.25) (layer F.Cu) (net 19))
 (segment (start 149.86 127) (end 149.86 123.19) (width 0.25) (layer F.Cu) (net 19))
 (segment (start 163.83 122.0647) (end 165.2447 120.65) (width 0.25) (layer F.Cu) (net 19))
 (segment (start 152.1106 122.0647) (end 163.83 122.0647) (width 0.25) (layer F.Cu) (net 19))
 (segment (start 150.9853 123.19) (end 152.1106 122.0647) (width 0.25) (layer F.Cu) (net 19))
 (segment (start 149.86 123.19) (end 150.9853 123.19) (width 0.25) (layer F.Cu) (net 19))
 (segment (start 164.1194 116.9847) (end 165.2447 118.11) (width 0.25) (layer F.Cu) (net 21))
 (segment (start 145.338 116.9847) (end 164.1194 116.9847) (width 0.25) (layer F.Cu) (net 21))
 (segment (start 142.7473 114.394) (end 145.338 116.9847) (width 0.25) (layer F.Cu) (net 21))
 (segment (start 133.1833 114.394) (end 142.7473 114.394) (width 0.25) (layer F.Cu) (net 21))
 (segment (start 130.5482 117.0291) (end 133.1833 114.394) (width 0.25) (layer F.Cu) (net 21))
 (segment (start 130.5482 118.745) (end 130.5482 117.0291) (width 0.25) (layer F.Cu) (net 21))
 (segment (start 131.445 118.745) (end 130.5482 118.745) (width 0.25) (layer F.Cu) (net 21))
 (segment (start 166.37 118.11) (end 165.2447 118.11) (width 0.25) (layer F.Cu) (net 21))
 (segment (start 167.4953 115.6806) (end 167.4953 115.57) (width 0.25) (layer F.Cu) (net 23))
 (segment (start 175.0047 123.19) (end 167.4953 115.6806) (width 0.25) (layer F.Cu) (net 23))
 (segment (start 176.53 123.19) (end 175.0047 123.19) (width 0.25) (layer F.Cu) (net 23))
 (segment (start 166.37 115.57) (end 167.4953 115.57) (width 0.25) (layer F.Cu) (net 23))
 (segment (start 168.7653 114.3) (end 167.4953 113.03) (width 0.25) (layer F.Cu) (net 25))
 (segment (start 176.53 114.3) (end 168.7653 114.3) (width 0.25) (layer F.Cu) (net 25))
 (segment (start 166.37 113.03) (end 167.4953 113.03) (width 0.25) (layer F.Cu) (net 25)))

